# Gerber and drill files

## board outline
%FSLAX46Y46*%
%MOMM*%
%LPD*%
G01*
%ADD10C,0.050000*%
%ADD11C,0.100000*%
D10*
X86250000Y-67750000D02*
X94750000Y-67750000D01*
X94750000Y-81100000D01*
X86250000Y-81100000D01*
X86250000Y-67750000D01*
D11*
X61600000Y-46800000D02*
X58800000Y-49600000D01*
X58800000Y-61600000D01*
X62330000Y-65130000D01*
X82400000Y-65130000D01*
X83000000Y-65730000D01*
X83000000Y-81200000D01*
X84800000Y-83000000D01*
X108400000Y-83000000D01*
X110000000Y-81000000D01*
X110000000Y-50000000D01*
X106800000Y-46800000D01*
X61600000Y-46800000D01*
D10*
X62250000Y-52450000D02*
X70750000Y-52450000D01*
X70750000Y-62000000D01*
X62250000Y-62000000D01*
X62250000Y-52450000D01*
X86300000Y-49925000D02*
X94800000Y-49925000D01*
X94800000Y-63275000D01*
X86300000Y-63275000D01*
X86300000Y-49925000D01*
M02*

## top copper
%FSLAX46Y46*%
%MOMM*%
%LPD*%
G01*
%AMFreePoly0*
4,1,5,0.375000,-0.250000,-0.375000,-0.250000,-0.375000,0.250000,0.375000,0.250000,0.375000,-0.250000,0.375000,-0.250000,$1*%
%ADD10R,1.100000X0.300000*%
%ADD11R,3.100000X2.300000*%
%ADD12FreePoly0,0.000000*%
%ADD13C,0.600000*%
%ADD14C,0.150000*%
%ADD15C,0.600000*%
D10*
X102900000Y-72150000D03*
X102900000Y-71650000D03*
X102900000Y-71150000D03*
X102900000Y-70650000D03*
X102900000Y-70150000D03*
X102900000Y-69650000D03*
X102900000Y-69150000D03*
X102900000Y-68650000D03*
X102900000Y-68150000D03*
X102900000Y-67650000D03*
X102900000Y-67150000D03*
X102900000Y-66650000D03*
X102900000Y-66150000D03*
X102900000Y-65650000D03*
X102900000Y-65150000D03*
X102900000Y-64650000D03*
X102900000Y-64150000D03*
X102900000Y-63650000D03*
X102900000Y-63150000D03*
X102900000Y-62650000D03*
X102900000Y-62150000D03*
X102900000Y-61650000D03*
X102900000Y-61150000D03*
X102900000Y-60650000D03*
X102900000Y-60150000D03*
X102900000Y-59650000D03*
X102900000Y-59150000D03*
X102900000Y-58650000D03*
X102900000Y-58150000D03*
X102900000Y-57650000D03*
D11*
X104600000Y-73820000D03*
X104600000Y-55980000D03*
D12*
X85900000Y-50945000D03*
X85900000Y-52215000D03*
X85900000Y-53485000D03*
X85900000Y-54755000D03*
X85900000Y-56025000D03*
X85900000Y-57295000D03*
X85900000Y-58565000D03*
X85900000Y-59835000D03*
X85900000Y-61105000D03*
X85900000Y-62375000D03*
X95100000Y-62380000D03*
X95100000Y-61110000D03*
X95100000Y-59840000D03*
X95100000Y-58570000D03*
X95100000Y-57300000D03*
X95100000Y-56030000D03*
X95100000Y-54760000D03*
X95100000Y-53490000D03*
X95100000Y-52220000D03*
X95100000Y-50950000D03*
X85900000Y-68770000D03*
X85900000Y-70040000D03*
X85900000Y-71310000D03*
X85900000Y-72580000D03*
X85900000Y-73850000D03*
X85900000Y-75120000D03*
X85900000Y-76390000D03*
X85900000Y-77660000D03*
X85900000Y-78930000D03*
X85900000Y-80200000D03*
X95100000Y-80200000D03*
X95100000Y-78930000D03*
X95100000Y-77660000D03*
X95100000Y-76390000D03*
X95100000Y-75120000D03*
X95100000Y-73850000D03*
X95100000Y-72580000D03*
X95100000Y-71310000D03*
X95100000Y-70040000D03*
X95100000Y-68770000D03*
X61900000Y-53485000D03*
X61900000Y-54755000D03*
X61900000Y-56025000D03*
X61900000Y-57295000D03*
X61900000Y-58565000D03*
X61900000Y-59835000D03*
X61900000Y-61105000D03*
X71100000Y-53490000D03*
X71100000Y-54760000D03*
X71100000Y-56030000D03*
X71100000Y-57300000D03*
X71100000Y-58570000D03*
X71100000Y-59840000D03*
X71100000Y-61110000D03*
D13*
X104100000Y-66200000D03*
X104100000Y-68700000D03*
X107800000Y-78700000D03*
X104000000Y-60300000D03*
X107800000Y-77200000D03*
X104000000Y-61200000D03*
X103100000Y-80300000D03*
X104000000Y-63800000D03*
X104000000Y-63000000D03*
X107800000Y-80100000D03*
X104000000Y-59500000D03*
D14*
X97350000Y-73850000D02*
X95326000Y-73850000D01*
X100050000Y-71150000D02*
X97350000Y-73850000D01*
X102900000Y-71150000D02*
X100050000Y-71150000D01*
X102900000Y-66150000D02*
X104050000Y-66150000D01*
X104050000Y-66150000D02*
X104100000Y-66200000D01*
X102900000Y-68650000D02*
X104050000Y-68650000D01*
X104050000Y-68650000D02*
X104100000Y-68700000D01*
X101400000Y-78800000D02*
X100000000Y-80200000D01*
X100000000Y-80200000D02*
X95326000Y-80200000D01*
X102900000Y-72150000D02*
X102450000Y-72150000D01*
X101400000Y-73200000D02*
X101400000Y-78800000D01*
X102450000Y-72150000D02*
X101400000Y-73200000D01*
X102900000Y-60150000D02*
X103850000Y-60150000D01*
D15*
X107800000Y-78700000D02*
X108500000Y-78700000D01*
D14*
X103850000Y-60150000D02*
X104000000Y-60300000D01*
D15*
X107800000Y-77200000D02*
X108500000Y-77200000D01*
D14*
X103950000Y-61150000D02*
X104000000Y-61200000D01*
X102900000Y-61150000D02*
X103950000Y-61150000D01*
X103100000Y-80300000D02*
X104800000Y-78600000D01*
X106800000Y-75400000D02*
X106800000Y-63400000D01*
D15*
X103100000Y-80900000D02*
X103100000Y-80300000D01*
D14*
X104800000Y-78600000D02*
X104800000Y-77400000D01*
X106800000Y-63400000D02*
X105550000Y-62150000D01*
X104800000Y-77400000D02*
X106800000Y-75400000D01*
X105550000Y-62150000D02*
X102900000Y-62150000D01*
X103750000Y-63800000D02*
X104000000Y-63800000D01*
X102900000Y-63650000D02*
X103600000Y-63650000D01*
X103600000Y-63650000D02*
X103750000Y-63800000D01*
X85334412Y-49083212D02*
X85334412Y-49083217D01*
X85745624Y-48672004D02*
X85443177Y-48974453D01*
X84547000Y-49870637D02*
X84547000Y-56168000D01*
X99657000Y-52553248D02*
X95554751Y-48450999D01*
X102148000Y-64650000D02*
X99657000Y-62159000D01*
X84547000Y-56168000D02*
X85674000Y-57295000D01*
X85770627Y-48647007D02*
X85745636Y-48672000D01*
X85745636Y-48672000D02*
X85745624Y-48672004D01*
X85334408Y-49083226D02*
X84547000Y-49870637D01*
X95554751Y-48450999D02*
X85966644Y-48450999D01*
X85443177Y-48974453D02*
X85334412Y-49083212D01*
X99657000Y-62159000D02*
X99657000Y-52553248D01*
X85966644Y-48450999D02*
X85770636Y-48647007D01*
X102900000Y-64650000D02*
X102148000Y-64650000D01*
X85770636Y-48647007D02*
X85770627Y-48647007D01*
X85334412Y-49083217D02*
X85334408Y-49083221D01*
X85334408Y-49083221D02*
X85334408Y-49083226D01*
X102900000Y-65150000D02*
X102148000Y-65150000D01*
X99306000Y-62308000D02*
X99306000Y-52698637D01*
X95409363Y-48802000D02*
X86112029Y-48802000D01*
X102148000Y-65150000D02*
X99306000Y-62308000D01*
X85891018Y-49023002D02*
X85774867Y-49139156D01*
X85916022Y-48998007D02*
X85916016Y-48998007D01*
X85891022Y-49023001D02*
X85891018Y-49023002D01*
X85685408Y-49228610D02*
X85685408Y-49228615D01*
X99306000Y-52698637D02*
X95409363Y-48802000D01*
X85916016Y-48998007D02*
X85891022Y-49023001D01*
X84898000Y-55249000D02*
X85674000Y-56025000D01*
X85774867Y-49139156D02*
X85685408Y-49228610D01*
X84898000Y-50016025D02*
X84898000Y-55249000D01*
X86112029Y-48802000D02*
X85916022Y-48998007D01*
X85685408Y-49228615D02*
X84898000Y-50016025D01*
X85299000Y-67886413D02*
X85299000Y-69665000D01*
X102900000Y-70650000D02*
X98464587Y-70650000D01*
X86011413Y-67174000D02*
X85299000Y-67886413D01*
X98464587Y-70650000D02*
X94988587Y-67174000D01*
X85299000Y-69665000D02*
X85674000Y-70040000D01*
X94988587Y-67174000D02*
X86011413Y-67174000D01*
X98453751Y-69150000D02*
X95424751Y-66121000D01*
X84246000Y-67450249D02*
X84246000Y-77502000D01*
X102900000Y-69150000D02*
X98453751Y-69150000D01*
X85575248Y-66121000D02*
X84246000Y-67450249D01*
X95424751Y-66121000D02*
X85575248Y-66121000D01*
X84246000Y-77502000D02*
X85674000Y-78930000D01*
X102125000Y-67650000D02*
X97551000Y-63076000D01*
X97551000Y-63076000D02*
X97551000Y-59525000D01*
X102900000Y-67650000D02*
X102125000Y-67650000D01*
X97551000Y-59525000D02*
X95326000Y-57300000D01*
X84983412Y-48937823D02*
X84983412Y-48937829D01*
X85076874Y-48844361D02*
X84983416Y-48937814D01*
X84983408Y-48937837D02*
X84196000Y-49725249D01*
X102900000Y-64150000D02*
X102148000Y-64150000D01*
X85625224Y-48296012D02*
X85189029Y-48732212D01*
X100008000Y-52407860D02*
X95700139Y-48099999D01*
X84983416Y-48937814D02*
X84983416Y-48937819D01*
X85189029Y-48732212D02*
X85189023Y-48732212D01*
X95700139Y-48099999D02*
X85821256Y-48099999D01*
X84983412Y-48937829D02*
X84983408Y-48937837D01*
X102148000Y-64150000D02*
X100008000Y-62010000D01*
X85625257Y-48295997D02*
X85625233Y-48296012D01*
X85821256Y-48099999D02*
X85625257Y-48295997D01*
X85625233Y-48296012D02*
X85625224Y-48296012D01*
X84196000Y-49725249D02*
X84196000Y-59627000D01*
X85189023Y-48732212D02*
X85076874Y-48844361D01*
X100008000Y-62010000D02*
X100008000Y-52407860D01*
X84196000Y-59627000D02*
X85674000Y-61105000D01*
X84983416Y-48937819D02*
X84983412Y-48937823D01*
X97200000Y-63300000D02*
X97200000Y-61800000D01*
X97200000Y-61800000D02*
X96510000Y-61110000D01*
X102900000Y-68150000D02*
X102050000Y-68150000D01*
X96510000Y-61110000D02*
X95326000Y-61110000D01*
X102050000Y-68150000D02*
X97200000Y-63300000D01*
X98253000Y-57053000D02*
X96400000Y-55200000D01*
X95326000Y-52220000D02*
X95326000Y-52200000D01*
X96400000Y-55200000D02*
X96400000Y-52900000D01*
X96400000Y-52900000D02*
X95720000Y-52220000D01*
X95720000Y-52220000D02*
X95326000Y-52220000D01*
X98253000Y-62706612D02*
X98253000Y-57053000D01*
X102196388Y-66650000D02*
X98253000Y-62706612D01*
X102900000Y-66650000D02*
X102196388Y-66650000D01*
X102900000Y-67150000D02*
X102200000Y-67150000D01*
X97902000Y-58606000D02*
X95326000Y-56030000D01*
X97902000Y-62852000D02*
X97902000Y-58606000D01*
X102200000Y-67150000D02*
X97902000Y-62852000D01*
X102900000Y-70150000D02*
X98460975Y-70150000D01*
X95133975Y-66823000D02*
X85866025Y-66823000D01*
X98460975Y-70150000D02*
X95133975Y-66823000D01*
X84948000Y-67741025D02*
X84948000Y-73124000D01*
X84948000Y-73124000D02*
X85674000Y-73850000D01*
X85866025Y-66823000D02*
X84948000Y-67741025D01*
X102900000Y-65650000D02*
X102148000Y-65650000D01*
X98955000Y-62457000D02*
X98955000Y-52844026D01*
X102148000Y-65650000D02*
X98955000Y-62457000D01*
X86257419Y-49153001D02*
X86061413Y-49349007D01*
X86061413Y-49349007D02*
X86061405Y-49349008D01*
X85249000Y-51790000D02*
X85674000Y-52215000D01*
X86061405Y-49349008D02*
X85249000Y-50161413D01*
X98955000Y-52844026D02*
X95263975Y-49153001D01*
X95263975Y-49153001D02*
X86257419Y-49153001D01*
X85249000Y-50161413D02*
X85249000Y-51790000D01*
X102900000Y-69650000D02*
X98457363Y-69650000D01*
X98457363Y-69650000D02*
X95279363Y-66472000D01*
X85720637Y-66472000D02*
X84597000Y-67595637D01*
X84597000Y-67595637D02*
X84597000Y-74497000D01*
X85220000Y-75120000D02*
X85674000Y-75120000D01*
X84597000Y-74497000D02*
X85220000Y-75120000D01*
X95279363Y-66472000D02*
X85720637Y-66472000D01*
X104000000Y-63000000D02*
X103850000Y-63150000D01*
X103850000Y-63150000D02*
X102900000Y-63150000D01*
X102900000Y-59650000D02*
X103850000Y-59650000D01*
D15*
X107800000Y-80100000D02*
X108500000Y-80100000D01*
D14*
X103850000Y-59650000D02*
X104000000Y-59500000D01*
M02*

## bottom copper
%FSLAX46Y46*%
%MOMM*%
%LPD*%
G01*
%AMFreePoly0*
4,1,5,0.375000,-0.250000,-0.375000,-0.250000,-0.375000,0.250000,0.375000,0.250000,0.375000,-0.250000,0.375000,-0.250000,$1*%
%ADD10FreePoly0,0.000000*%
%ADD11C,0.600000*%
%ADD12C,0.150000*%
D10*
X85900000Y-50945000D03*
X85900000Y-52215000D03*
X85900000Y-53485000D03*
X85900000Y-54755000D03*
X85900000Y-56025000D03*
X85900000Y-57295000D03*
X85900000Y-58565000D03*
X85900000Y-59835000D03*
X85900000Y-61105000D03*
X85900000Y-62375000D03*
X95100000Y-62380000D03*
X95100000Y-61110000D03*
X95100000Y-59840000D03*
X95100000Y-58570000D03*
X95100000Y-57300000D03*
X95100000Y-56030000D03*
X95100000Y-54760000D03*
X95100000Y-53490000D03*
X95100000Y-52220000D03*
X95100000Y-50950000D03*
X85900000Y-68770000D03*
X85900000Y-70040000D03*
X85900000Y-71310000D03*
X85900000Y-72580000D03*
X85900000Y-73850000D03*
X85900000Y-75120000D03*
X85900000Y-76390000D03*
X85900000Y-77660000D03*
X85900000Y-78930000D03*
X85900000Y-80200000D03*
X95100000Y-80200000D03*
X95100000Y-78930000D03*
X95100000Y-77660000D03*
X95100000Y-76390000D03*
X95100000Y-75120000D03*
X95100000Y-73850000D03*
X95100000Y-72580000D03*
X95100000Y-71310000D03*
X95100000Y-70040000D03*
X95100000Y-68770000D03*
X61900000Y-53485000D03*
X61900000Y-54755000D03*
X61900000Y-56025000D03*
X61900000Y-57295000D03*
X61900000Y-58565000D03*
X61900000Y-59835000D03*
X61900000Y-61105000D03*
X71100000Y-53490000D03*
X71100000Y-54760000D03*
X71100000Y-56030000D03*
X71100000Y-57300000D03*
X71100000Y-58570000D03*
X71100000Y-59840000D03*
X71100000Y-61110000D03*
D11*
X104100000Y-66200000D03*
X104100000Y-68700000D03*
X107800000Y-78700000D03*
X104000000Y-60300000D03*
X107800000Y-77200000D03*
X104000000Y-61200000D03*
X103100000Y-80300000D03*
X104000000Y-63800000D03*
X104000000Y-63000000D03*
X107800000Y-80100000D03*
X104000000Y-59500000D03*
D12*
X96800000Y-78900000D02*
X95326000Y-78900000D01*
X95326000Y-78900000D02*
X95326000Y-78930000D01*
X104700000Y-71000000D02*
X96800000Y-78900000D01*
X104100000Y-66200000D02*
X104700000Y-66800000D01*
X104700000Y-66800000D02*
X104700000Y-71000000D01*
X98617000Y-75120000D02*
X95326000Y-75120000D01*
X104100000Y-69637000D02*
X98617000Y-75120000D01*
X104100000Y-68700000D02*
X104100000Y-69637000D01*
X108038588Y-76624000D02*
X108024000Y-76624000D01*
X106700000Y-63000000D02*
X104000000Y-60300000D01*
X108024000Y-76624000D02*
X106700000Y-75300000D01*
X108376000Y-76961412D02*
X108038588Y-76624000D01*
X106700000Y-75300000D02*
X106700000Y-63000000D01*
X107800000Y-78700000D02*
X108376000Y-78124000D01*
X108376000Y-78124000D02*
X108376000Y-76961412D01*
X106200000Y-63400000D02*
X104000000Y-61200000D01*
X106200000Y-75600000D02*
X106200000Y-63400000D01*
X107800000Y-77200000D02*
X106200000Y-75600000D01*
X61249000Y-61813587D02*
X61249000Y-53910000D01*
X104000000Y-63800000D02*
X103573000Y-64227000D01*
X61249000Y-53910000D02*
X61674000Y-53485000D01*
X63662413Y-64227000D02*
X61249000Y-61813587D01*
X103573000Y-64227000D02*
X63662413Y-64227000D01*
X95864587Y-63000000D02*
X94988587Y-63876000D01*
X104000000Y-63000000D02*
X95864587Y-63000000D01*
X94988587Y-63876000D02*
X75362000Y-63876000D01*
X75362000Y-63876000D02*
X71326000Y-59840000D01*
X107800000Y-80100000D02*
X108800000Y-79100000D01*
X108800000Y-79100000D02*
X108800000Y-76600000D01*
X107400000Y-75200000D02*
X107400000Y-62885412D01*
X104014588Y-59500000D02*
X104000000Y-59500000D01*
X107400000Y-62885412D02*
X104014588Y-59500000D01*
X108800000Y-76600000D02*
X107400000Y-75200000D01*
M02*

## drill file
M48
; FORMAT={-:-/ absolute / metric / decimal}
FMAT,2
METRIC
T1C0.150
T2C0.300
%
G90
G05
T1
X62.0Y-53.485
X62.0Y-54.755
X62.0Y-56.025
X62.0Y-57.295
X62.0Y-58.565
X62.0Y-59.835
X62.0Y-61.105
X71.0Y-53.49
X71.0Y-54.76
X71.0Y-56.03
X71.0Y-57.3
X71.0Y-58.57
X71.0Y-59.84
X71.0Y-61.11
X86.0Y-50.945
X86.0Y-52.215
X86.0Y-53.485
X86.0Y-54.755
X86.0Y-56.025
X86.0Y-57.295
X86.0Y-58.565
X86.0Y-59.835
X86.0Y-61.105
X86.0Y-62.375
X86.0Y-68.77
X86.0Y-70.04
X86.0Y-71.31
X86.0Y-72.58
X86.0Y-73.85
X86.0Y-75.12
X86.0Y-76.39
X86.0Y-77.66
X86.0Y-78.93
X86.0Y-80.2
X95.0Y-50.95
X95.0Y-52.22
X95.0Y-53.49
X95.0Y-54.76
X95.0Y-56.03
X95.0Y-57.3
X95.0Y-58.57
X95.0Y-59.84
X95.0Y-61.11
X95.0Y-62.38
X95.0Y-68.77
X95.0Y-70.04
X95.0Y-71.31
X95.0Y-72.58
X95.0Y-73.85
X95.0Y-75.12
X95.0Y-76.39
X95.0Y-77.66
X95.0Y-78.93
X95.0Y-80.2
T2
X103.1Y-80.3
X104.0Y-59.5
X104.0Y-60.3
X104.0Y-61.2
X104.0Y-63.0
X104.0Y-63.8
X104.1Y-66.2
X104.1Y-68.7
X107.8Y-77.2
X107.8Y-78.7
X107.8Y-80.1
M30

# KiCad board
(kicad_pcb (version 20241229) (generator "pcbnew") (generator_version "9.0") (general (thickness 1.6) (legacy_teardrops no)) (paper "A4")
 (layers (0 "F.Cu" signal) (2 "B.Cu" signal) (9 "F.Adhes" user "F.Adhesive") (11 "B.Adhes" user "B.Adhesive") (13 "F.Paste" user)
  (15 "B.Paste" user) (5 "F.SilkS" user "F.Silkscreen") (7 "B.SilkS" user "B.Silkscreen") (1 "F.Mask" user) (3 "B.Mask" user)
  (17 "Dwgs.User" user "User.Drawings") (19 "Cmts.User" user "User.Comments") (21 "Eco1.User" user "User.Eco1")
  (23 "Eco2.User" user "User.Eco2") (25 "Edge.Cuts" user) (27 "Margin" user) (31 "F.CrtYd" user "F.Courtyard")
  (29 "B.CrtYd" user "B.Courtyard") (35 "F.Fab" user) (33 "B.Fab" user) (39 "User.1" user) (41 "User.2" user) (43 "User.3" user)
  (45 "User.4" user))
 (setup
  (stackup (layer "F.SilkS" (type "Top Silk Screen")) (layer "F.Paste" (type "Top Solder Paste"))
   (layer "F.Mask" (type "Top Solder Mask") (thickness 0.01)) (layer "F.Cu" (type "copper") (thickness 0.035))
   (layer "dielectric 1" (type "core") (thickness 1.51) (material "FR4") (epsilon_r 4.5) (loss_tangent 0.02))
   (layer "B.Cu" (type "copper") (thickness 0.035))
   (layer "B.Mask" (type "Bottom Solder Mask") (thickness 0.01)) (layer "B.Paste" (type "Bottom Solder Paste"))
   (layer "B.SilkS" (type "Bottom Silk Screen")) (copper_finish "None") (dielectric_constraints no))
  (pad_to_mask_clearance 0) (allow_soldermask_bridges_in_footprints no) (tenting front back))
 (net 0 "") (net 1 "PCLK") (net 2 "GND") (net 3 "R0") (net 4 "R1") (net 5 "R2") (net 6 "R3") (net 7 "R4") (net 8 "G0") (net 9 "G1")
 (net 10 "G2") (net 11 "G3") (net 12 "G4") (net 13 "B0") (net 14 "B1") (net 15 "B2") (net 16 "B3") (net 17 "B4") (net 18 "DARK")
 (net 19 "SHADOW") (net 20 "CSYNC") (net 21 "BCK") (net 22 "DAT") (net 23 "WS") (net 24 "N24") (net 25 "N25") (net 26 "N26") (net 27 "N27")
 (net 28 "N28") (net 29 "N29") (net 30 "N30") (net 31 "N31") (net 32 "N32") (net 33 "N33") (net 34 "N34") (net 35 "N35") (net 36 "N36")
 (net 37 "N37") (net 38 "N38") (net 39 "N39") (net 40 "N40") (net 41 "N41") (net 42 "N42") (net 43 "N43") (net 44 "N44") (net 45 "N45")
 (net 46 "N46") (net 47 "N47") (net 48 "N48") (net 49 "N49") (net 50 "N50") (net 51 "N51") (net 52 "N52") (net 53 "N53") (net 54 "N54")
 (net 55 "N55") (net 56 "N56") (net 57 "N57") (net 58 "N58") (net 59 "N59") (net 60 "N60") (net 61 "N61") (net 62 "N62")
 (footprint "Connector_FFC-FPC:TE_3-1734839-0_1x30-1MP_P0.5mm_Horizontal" (layer "F.Cu") (at 104.25 64.9 90)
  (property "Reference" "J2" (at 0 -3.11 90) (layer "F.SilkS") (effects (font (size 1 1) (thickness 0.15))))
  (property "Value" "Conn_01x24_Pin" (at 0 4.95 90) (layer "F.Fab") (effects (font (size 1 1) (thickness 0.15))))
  (pad "1" smd rect (at -7.25 -1.35 90) (size 0.3 1.1) (layers "F.Cu" "F.Mask" "F.Paste") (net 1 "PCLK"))
  (pad "2" smd rect (at -6.75 -1.35 90) (size 0.3 1.1) (layers "F.Cu" "F.Mask" "F.Paste") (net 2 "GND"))
  (pad "3" smd rect (at -6.25 -1.35 90) (size 0.3 1.1) (layers "F.Cu" "F.Mask" "F.Paste") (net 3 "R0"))
  (pad "4" smd rect (at -5.75 -1.35 90) (size 0.3 1.1) (layers "F.Cu" "F.Mask" "F.Paste") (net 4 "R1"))
  (pad "5" smd rect (at -5.25 -1.35 90) (size 0.3 1.1) (layers "F.Cu" "F.Mask" "F.Paste") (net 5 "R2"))
  (pad "6" smd rect (at -4.75 -1.35 90) (size 0.3 1.1) (layers "F.Cu" "F.Mask" "F.Paste") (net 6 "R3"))
  (pad "7" smd rect (at -4.25 -1.35 90) (size 0.3 1.1) (layers "F.Cu" "F.Mask" "F.Paste") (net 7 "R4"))
  (pad "8" smd rect (at -3.75 -1.35 90) (size 0.3 1.1) (layers "F.Cu" "F.Mask" "F.Paste") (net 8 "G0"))
  (pad "9" smd rect (at -3.25 -1.35 90) (size 0.3 1.1) (layers "F.Cu" "F.Mask" "F.Paste") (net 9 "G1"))
  (pad "10" smd rect (at -2.75 -1.35 90) (size 0.3 1.1) (layers "F.Cu" "F.Mask" "F.Paste") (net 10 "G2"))
  (pad "11" smd rect (at -2.25 -1.35 90) (size 0.3 1.1) (layers "F.Cu" "F.Mask" "F.Paste") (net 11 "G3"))
  (pad "12" smd rect (at -1.75 -1.35 90) (size 0.3 1.1) (layers "F.Cu" "F.Mask" "F.Paste") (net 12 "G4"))
  (pad "13" smd rect (at -1.25 -1.35 90) (size 0.3 1.1) (layers "F.Cu" "F.Mask" "F.Paste") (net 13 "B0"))
  (pad "14" smd rect (at -0.75 -1.35 90) (size 0.3 1.1) (layers "F.Cu" "F.Mask" "F.Paste") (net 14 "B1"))
  (pad "15" smd rect (at -0.25 -1.35 90) (size 0.3 1.1) (layers "F.Cu" "F.Mask" "F.Paste") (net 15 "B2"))
  (pad "16" smd rect (at 0.25 -1.35 90) (size 0.3 1.1) (layers "F.Cu" "F.Mask" "F.Paste") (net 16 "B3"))
  (pad "17" smd rect (at 0.75 -1.35 90) (size 0.3 1.1) (layers "F.Cu" "F.Mask" "F.Paste") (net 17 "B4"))
  (pad "18" smd rect (at 1.25 -1.35 90) (size 0.3 1.1) (layers "F.Cu" "F.Mask" "F.Paste") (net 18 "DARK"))
  (pad "19" smd rect (at 1.75 -1.35 90) (size 0.3 1.1) (layers "F.Cu" "F.Mask" "F.Paste") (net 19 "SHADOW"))
  (pad "20" smd rect (at 2.25 -1.35 90) (size 0.3 1.1) (layers "F.Cu" "F.Mask" "F.Paste") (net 2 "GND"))
  (pad "21" smd rect (at 2.75 -1.35 90) (size 0.3 1.1) (layers "F.Cu" "F.Mask" "F.Paste") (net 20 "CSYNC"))
  (pad "22" smd rect (at 3.25 -1.35 90) (size 0.3 1.1) (layers "F.Cu" "F.Mask" "F.Paste") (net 2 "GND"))
  (pad "23" smd rect (at 3.75 -1.35 90) (size 0.3 1.1) (layers "F.Cu" "F.Mask" "F.Paste") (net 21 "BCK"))
  (pad "24" smd rect (at 4.25 -1.35 90) (size 0.3 1.1) (layers "F.Cu" "F.Mask" "F.Paste") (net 2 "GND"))
  (pad "25" smd rect (at 4.75 -1.35 90) (size 0.3 1.1) (layers "F.Cu" "F.Mask" "F.Paste") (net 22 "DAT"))
  (pad "26" smd rect (at 5.25 -1.35 90) (size 0.3 1.1) (layers "F.Cu" "F.Mask" "F.Paste") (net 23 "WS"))
  (pad "27" smd rect (at 5.75 -1.35 90) (size 0.3 1.1) (layers "F.Cu" "F.Mask" "F.Paste") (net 2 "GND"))
  (pad "28" smd rect (at 6.25 -1.35 90) (size 0.3 1.1) (layers "F.Cu" "F.Mask" "F.Paste") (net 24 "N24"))
  (pad "29" smd rect (at 6.75 -1.35 90) (size 0.3 1.1) (layers "F.Cu" "F.Mask" "F.Paste") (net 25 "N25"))
  (pad "30" smd rect (at 7.25 -1.35 90) (size 0.3 1.1) (layers "F.Cu" "F.Mask" "F.Paste") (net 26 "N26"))
  (pad "MP" smd rect (at -8.92 0.35 90) (size 2.3 3.1) (layers "F.Cu" "F.Mask" "F.Paste"))
  (pad "MP" smd rect (at 8.92 0.35 90) (size 2.3 3.1) (layers "F.Cu" "F.Mask" "F.Paste")))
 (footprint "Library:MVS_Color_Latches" (layer "F.Cu") (at 77.8 65.43)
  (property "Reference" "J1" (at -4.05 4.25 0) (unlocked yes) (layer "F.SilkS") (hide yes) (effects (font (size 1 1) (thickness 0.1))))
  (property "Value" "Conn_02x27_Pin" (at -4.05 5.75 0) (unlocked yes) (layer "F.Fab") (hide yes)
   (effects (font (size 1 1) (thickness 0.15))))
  (pad "1" thru_hole custom (at 8.2 -14.485) (size 0.75 0.5) (drill 0.15 (offset -0.1 0)) (layers "*.Cu" "*.Mask") (remove_unused_layers no)
   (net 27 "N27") (options (clearance outline) (anchor rect)) (primitives))
  (pad "2" thru_hole custom (at 8.2 -13.215) (size 0.75 0.5) (drill 0.15 (offset -0.1 0)) (layers "*.Cu" "*.Mask") (remove_unused_layers no)
   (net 14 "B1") (options (clearance outline) (anchor rect)) (primitives))
  (pad "3" thru_hole custom (at 8.2 -11.945) (size 0.75 0.5) (drill 0.15 (offset -0.1 0)) (layers "*.Cu" "*.Mask") (remove_unused_layers no)
   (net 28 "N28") (options (clearance outline) (anchor rect)) (primitives))
  (pad "4" thru_hole custom (at 8.2 -10.675) (size 0.75 0.5) (drill 0.15 (offset -0.1 0)) (layers "*.Cu" "*.Mask") (remove_unused_layers no)
   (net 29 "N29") (options (clearance outline) (anchor rect)) (primitives))
  (pad "5" thru_hole custom (at 8.2 -9.405) (size 0.75 0.5) (drill 0.15 (offset -0.1 0)) (layers "*.Cu" "*.Mask") (remove_unused_layers no)
   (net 15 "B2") (options (clearance outline) (anchor rect)) (primitives))
  (pad "6" thru_hole custom (at 8.2 -8.135) (size 0.75 0.5) (drill 0.15 (offset -0.1 0)) (layers "*.Cu" "*.Mask") (remove_unused_layers no)
   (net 16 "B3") (options (clearance outline) (anchor rect)) (primitives))
  (pad "7" thru_hole custom (at 8.2 -6.865) (size 0.75 0.5) (drill 0.15 (offset -0.1 0)) (layers "*.Cu" "*.Mask") (remove_unused_layers no)
   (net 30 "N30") (options (clearance outline) (anchor rect)) (primitives))
  (pad "8" thru_hole custom (at 8.2 -5.595) (size 0.75 0.5) (drill 0.15 (offset -0.1 0)) (layers "*.Cu" "*.Mask") (remove_unused_layers no)
   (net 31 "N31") (options (clearance outline) (anchor rect)) (primitives))
  (pad "9" thru_hole custom (at 8.2 -4.325) (size 0.75 0.5) (drill 0.15 (offset -0.1 0)) (layers "*.Cu" "*.Mask") (remove_unused_layers no)
   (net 17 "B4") (options (clearance outline) (anchor rect)) (primitives))
  (pad "10" thru_hole custom (at 8.2 -3.055) (size 0.75 0.5) (drill 0.15 (offset -0.1 0)) (layers "*.Cu" "*.Mask") (remove_unused_layers no)
   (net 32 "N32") (options (clearance outline) (anchor rect)) (primitives))
  (pad "11" thru_hole custom (at 17.2 -3.05) (size 0.75 0.5) (drill 0.15 (offset 0.1 0)) (layers "*.Cu" "*.Mask") (remove_unused_layers no)
   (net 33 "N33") (options (clearance outline) (anchor rect)) (primitives))
  (pad "12" thru_hole custom (at 17.2 -4.32) (size 0.75 0.5) (drill 0.15 (offset 0.1 0)) (layers "*.Cu" "*.Mask") (remove_unused_layers no)
   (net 9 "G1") (options (clearance outline) (anchor rect)) (primitives))
  (pad "13" thru_hole custom (at 17.2 -5.59) (size 0.75 0.5) (drill 0.15 (offset 0.1 0)) (layers "*.Cu" "*.Mask") (remove_unused_layers no)
   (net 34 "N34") (options (clearance outline) (anchor rect)) (primitives))
  (pad "14" thru_hole custom (at 17.2 -6.86) (size 0.75 0.5) (drill 0.15 (offset 0.1 0)) (layers "*.Cu" "*.Mask") (remove_unused_layers no)
   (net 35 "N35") (options (clearance outline) (anchor rect)) (primitives))
  (pad "15" thru_hole custom (at 17.2 -8.13) (size 0.75 0.5) (drill 0.15 (offset 0.1 0)) (layers "*.Cu" "*.Mask") (remove_unused_layers no)
   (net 10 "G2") (options (clearance outline) (anchor rect)) (primitives))
  (pad "16" thru_hole custom (at 17.2 -9.4) (size 0.75 0.5) (drill 0.15 (offset 0.1 0)) (layers "*.Cu" "*.Mask") (remove_unused_layers no)
   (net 11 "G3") (options (clearance outline) (anchor rect)) (primitives))
  (pad "17" thru_hole custom (at 17.2 -10.67) (size 0.75 0.5) (drill 0.15 (offset 0.1 0)) (layers "*.Cu" "*.Mask") (remove_unused_layers no)
   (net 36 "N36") (options (clearance outline) (anchor rect)) (primitives))
  (pad "18" thru_hole custom (at 17.2 -11.94) (size 0.75 0.5) (drill 0.15 (offset 0.1 0)) (layers "*.Cu" "*.Mask") (remove_unused_layers no)
   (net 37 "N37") (options (clearance outline) (anchor rect)) (primitives))
  (pad "19" thru_hole custom (at 17.2 -13.21) (size 0.75 0.5) (drill 0.15 (offset 0.1 0)) (layers "*.Cu" "*.Mask") (remove_unused_layers no)
   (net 12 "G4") (options (clearance outline) (anchor rect)) (primitives))
  (pad "20" thru_hole custom (at 17.2 -14.48) (size 0.75 0.5) (drill 0.15 (offset 0.1 0)) (layers "*.Cu" "*.Mask") (remove_unused_layers no)
   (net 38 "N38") (options (clearance outline) (anchor rect)) (primitives))
  (pad "21" thru_hole custom (at 8.2 3.34) (size 0.75 0.5) (drill 0.15 (offset -0.1 0)) (layers "*.Cu" "*.Mask") (remove_unused_layers no)
   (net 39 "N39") (options (clearance outline) (anchor rect)) (primitives))
  (pad "22" thru_hole custom (at 8.2 4.61) (size 0.75 0.5) (drill 0.15 (offset -0.1 0)) (layers "*.Cu" "*.Mask") (remove_unused_layers no)
   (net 4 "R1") (options (clearance outline) (anchor rect)) (primitives))
  (pad "23" thru_hole custom (at 8.2 5.88) (size 0.75 0.5) (drill 0.15 (offset -0.1 0)) (layers "*.Cu" "*.Mask") (remove_unused_layers no)
   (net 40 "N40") (options (clearance outline) (anchor rect)) (primitives))
  (pad "24" thru_hole custom (at 8.2 7.15) (size 0.75 0.5) (drill 0.15 (offset -0.1 0)) (layers "*.Cu" "*.Mask") (remove_unused_layers no)
   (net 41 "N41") (options (clearance outline) (anchor rect)) (primitives))
  (pad "25" thru_hole custom (at 8.2 8.42) (size 0.75 0.5) (drill 0.15 (offset -0.1 0)) (layers "*.Cu" "*.Mask") (remove_unused_layers no)
   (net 5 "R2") (options (clearance outline) (anchor rect)) (primitives))
  (pad "26" thru_hole custom (at 8.2 9.69) (size 0.75 0.5) (drill 0.15 (offset -0.1 0)) (layers "*.Cu" "*.Mask") (remove_unused_layers no)
   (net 6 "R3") (options (clearance outline) (anchor rect)) (primitives))
  (pad "27" thru_hole custom (at 8.2 10.96) (size 0.75 0.5) (drill 0.15 (offset -0.1 0)) (layers "*.Cu" "*.Mask") (remove_unused_layers no)
   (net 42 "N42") (options (clearance outline) (anchor rect)) (primitives))
  (pad "28" thru_hole custom (at 8.2 12.23) (size 0.75 0.5) (drill 0.15 (offset -0.1 0)) (layers "*.Cu" "*.Mask") (remove_unused_layers no)
   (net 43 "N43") (options (clearance outline) (anchor rect)) (primitives))
  (pad "29" thru_hole custom (at 8.2 13.5) (size 0.75 0.5) (drill 0.15 (offset -0.1 0)) (layers "*.Cu" "*.Mask") (remove_unused_layers no)
   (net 7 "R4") (options (clearance outline) (anchor rect)) (primitives))
  (pad "30" thru_hole custom (at 8.2 14.77) (size 0.75 0.5) (drill 0.15 (offset -0.1 0)) (layers "*.Cu" "*.Mask") (remove_unused_layers no)
   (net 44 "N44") (options (clearance outline) (anchor rect)) (primitives))
  (pad "31" thru_hole custom (at 17.2 14.77) (size 0.75 0.5) (drill 0.15 (offset 0.1 0)) (layers "*.Cu" "*.Mask") (remove_unused_layers no)
   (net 1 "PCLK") (options (clearance outline) (anchor rect)) (primitives))
  (pad "32" thru_hole custom (at 17.2 13.5) (size 0.75 0.5) (drill 0.15 (offset 0.1 0)) (layers "*.Cu" "*.Mask") (remove_unused_layers no)
   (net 13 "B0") (options (clearance outline) (anchor rect)) (primitives))
  (pad "33" thru_hole custom (at 17.2 12.23) (size 0.75 0.5) (drill 0.15 (offset 0.1 0)) (layers "*.Cu" "*.Mask") (remove_unused_layers no)
   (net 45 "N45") (options (clearance outline) (anchor rect)) (primitives))
  (pad "34" thru_hole custom (at 17.2 10.96) (size 0.75 0.5) (drill 0.15 (offset 0.1 0)) (layers "*.Cu" "*.Mask") (remove_unused_layers no)
   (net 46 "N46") (options (clearance outline) (anchor rect)) (primitives))
  (pad "35" thru_hole custom (at 17.2 9.69) (size 0.75 0.5) (drill 0.15 (offset 0.1 0)) (layers "*.Cu" "*.Mask") (remove_unused_layers no)
   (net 8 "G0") (options (clearance outline) (anchor rect)) (primitives))
  (pad "36" thru_hole custom (at 17.2 8.42) (size 0.75 0.5) (drill 0.15 (offset 0.1 0)) (layers "*.Cu" "*.Mask") (remove_unused_layers no)
   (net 3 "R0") (options (clearance outline) (anchor rect)) (primitives))
  (pad "37" thru_hole custom (at 17.2 7.15) (size 0.75 0.5) (drill 0.15 (offset 0.1 0)) (layers "*.Cu" "*.Mask") (remove_unused_layers no)
   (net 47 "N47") (options (clearance outline) (anchor rect)) (primitives))
  (pad "38" thru_hole custom (at 17.2 5.88) (size 0.75 0.5) (drill 0.15 (offset 0.1 0)) (layers "*.Cu" "*.Mask") (remove_unused_layers no)
   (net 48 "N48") (options (clearance outline) (anchor rect)) (primitives))
  (pad "39" thru_hole custom (at 17.2 4.61) (size 0.75 0.5) (drill 0.15 (offset 0.1 0)) (layers "*.Cu" "*.Mask") (remove_unused_layers no)
   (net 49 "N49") (options (clearance outline) (anchor rect)) (primitives))
  (pad "40" thru_hole custom (at 17.2 3.34) (size 0.75 0.5) (drill 0.15 (offset 0.1 0)) (layers "*.Cu" "*.Mask") (remove_unused_layers no)
   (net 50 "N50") (options (clearance outline) (anchor rect)) (primitives))
  (pad "41" thru_hole custom (at -15.8 -11.945) (size 0.75 0.5) (drill 0.15 (offset -0.1 0)) (layers "*.Cu" "*.Mask")
   (remove_unused_layers no) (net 18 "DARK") (options (clearance outline) (anchor rect)) (primitives))
  (pad "42" thru_hole custom (at -15.8 -10.675) (size 0.75 0.5) (drill 0.15 (offset -0.1 0)) (layers "*.Cu" "*.Mask")
   (remove_unused_layers no) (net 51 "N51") (options (clearance outline) (anchor rect)) (primitives))
  (pad "43" thru_hole custom (at -15.8 -9.405) (size 0.75 0.5) (drill 0.15 (offset -0.1 0)) (layers "*.Cu" "*.Mask")
   (remove_unused_layers no) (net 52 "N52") (options (clearance outline) (anchor rect)) (primitives))
  (pad "44" thru_hole custom (at -15.8 -8.135) (size 0.75 0.5) (drill 0.15 (offset -0.1 0)) (layers "*.Cu" "*.Mask")
   (remove_unused_layers no) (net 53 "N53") (options (clearance outline) (anchor rect)) (primitives))
  (pad "45" thru_hole custom (at -15.8 -6.865) (size 0.75 0.5) (drill 0.15 (offset -0.1 0)) (layers "*.Cu" "*.Mask")
   (remove_unused_layers no) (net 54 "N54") (options (clearance outline) (anchor rect)) (primitives))
  (pad "46" thru_hole custom (at -15.8 -5.595) (size 0.75 0.5) (drill 0.15 (offset -0.1 0)) (layers "*.Cu" "*.Mask")
   (remove_unused_layers no) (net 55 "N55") (options (clearance outline) (anchor rect)) (primitives))
  (pad "47" thru_hole custom (at -15.8 -4.325) (size 0.75 0.5) (drill 0.15 (offset -0.1 0)) (layers "*.Cu" "*.Mask")
   (remove_unused_layers no) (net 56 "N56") (options (clearance outline) (anchor rect)) (primitives))
  (pad "48" thru_hole custom (at -6.8 -11.94) (size 0.75 0.5) (drill 0.15 (offset 0.1 0)) (layers "*.Cu" "*.Mask") (remove_unused_layers no)
   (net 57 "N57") (options (clearance outline) (anchor rect)) (primitives))
  (pad "49" thru_hole custom (at -6.8 -10.67) (size 0.75 0.5) (drill 0.15 (offset 0.1 0)) (layers "*.Cu" "*.Mask") (remove_unused_layers no)
   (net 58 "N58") (options (clearance outline) (anchor rect)) (primitives))
  (pad "50" thru_hole custom (at -6.8 -9.4) (size 0.75 0.5) (drill 0.15 (offset 0.1 0)) (layers "*.Cu" "*.Mask") (remove_unused_layers no)
   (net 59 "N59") (options (clearance outline) (anchor rect)) (primitives))
  (pad "51" thru_hole custom (at -6.8 -8.13) (size 0.75 0.5) (drill 0.15 (offset 0.1 0)) (layers "*.Cu" "*.Mask") (remove_unused_layers no)
   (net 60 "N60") (options (clearance outline) (anchor rect)) (primitives))
  (pad "52" thru_hole custom (at -6.8 -6.86) (size 0.75 0.5) (drill 0.15 (offset 0.1 0)) (layers "*.Cu" "*.Mask") (remove_unused_layers no)
   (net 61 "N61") (options (clearance outline) (anchor rect)) (primitives))
  (pad "53" thru_hole custom (at -6.8 -5.59) (size 0.75 0.5) (drill 0.15 (offset 0.1 0)) (layers "*.Cu" "*.Mask") (remove_unused_layers no)
   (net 19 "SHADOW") (options (clearance outline) (anchor rect)) (primitives))
  (pad "54" thru_hole custom (at -6.8 -4.32) (size 0.75 0.5) (drill 0.15 (offset 0.1 0)) (layers "*.Cu" "*.Mask") (remove_unused_layers no)
   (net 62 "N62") (options (clearance outline) (anchor rect)) (primitives)))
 (gr_rect (start 86.25 67.75) (end 94.75 81.1) (stroke (width 0.05) (type default)) (fill no) (layer "Edge.Cuts"))
 (gr_poly
  (pts (xy 61.6 46.8) (xy 58.8 49.6) (xy 58.8 61.6) (xy 62.33 65.13) (xy 82.4 65.13) (xy 83 65.73) (xy 83 81.2) (xy 84.8 83) (xy 108.4 83)
   (xy 110 81) (xy 110 50) (xy 106.8 46.8))
  (stroke (width 0.1) (type solid)) (fill no) (layer "Edge.Cuts"))
 (gr_rect (start 62.25 52.45) (end 70.75 62) (stroke (width 0.05) (type default)) (fill no) (layer "Edge.Cuts"))
 (gr_rect (start 86.3 49.925) (end 94.8 63.275) (stroke (width 0.05) (type default)) (fill no) (layer "Edge.Cuts"))
 (segment (start 97.35 73.85) (end 95.326 73.85) (width 0.15) (layer "F.Cu") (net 3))
 (segment (start 100.05 71.15) (end 97.35 73.85) (width 0.15) (layer "F.Cu") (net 3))
 (segment (start 102.9 71.15) (end 100.05 71.15) (width 0.15) (layer "F.Cu") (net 3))
 (segment (start 102.9 66.15) (end 104.05 66.15) (width 0.15) (layer "F.Cu") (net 13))
 (segment (start 104.05 66.15) (end 104.1 66.2) (width 0.15) (layer "F.Cu") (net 13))
 (via (at 104.1 66.2) (size 0.6) (drill 0.3) (layers "F.Cu" "B.Cu") (free yes) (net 13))
 (segment (start 96.8 78.9) (end 95.326 78.9) (width 0.15) (layer "B.Cu") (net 13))
 (segment (start 95.326 78.9) (end 95.326 78.93) (width 0.15) (layer "B.Cu") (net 13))
 (segment (start 104.7 71) (end 96.8 78.9) (width 0.15) (layer "B.Cu") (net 13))
 (segment (start 104.1 66.2) (end 104.7 66.8) (width 0.15) (layer "B.Cu") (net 13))
 (segment (start 104.7 66.8) (end 104.7 71) (width 0.15) (layer "B.Cu") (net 13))
 (segment (start 102.9 68.65) (end 104.05 68.65) (width 0.15) (layer "F.Cu") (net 8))
 (segment (start 104.05 68.65) (end 104.1 68.7) (width 0.15) (layer "F.Cu") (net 8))
 (via (at 104.1 68.7) (size 0.6) (drill 0.3) (layers "F.Cu" "B.Cu") (free yes) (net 8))
 (segment (start 98.617 75.12) (end 95.326 75.12) (width 0.15) (layer "B.Cu") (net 8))
 (segment (start 104.1 69.637) (end 98.617 75.12) (width 0.15) (layer "B.Cu") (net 8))
 (segment (start 104.1 68.7) (end 104.1 69.637) (width 0.15) (layer "B.Cu") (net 8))
 (segment (start 101.4 78.8) (end 100 80.2) (width 0.15) (layer "F.Cu") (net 1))
 (segment (start 100 80.2) (end 95.326 80.2) (width 0.15) (layer "F.Cu") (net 1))
 (segment (start 102.9 72.15) (end 102.45 72.15) (width 0.15) (layer "F.Cu") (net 1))
 (segment (start 101.4 73.2) (end 101.4 78.8) (width 0.15) (layer "F.Cu") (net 1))
 (segment (start 102.45 72.15) (end 101.4 73.2) (width 0.15) (layer "F.Cu") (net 1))
 (segment (start 102.9 60.15) (end 103.85 60.15) (width 0.15) (layer "F.Cu") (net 22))
 (segment (start 107.8 78.7) (end 108.5 78.7) (width 0.6) (layers "F.Cu" "F.Mask") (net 22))
 (segment (start 103.85 60.15) (end 104 60.3) (width 0.15) (layer "F.Cu") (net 22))
 (via (at 107.8 78.7) (size 0.6) (drill 0.3) (layers "F.Cu" "B.Cu") (free yes) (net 22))
 (via (at 104 60.3) (size 0.6) (drill 0.3) (layers "F.Cu" "B.Cu") (free yes) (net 22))
 (segment (start 108.038588 76.624) (end 108.024 76.624) (width 0.15) (layer "B.Cu") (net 22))
 (segment (start 106.7 63) (end 104 60.3) (width 0.15) (layer "B.Cu") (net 22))
 (segment (start 108.024 76.624) (end 106.7 75.3) (width 0.15) (layer "B.Cu") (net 22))
 (segment (start 108.376 76.961412) (end 108.038588 76.624) (width 0.15) (layer "B.Cu") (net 22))
 (segment (start 106.7 75.3) (end 106.7 63) (width 0.15) (layer "B.Cu") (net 22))
 (segment (start 107.8 78.7) (end 108.376 78.124) (width 0.15) (layer "B.Cu") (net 22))
 (segment (start 108.376 78.124) (end 108.376 76.961412) (width 0.15) (layer "B.Cu") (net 22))
 (segment (start 107.8 77.2) (end 108.5 77.2) (width 0.6) (layers "F.Cu" "F.Mask") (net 21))
 (segment (start 103.95 61.15) (end 104 61.2) (width 0.15) (layer "F.Cu") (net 21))
 (segment (start 102.9 61.15) (end 103.95 61.15) (width 0.15) (layer "F.Cu") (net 21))
 (via (at 107.8 77.2) (size 0.6) (drill 0.3) (layers "F.Cu" "B.Cu") (free yes) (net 21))
 (via (at 104 61.2) (size 0.6) (drill 0.3) (layers "F.Cu" "B.Cu") (free yes) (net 21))
 (segment (start 106.2 63.4) (end 104 61.2) (width 0.15) (layer "B.Cu") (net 21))
 (segment (start 106.2 75.6) (end 106.2 63.4) (width 0.15) (layer "B.Cu") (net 21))
 (segment (start 107.8 77.2) (end 106.2 75.6) (width 0.15) (layer "B.Cu") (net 21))
 (segment (start 103.1 80.3) (end 104.8 78.6) (width 0.15) (layer "F.Cu") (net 20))
 (segment (start 106.8 75.4) (end 106.8 63.4) (width 0.15) (layer "F.Cu") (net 20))
 (segment (start 103.1 80.9) (end 103.1 80.3) (width 0.6) (layer "F.Cu") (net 20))
 (segment (start 104.8 78.6) (end 104.8 77.4) (width 0.15) (layer "F.Cu") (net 20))
 (segment (start 106.8 63.4) (end 105.55 62.15) (width 0.15) (layer "F.Cu") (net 20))
 (segment (start 104.8 77.4) (end 106.8 75.4) (width 0.15) (layer "F.Cu") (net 20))
 (segment (start 105.55 62.15) (end 102.9 62.15) (width 0.15) (layer "F.Cu") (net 20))
 (via (at 103.1 80.3) (size 0.6) (drill 0.3) (layers "F.Cu" "B.Cu") (free yes) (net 20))
 (segment (start 103.75 63.8) (end 104 63.8) (width 0.15) (layer "F.Cu") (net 18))
 (segment (start 102.9 63.65) (end 103.6 63.65) (width 0.15) (layer "F.Cu") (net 18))
 (segment (start 103.6 63.65) (end 103.75 63.8) (width 0.15) (layer "F.Cu") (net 18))
 (via (at 104 63.8) (size 0.6) (drill 0.3) (layers "F.Cu" "B.Cu") (free yes) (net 18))
 (segment (start 61.249 61.813587) (end 61.249 53.91) (width 0.15) (layer "B.Cu") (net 18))
 (segment (start 104 63.8) (end 103.573 64.227) (width 0.15) (layer "B.Cu") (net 18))
 (segment (start 61.249 53.91) (end 61.674 53.485) (width 0.15) (layer "B.Cu") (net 18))
 (segment (start 63.662413 64.227) (end 61.249 61.813587) (width 0.15) (layer "B.Cu") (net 18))
 (segment (start 103.573 64.227) (end 63.662413 64.227) (width 0.15) (layer "B.Cu") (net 18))
 (segment (start 85.334412 49.083212) (end 85.334412 49.083217) (width 0.15) (layer "F.Cu") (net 16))
 (segment (start 85.745624 48.672004) (end 85.443177 48.974453) (width 0.15) (layer "F.Cu") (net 16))
 (segment (start 84.547 49.870637) (end 84.547 56.168) (width 0.15) (layer "F.Cu") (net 16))
 (segment (start 99.657 52.553248) (end 95.554751 48.450999) (width 0.15) (layer "F.Cu") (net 16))
 (segment (start 102.148 64.65) (end 99.657 62.159) (width 0.15) (layer "F.Cu") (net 16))
 (segment (start 84.547 56.168) (end 85.674 57.295) (width 0.15) (layer "F.Cu") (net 16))
 (segment (start 85.770627 48.647007) (end 85.745636 48.672) (width 0.15) (layer "F.Cu") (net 16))
 (segment (start 85.745636 48.672) (end 85.745624 48.672004) (width 0.15) (layer "F.Cu") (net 16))
 (segment (start 85.334408 49.083226) (end 84.547 49.870637) (width 0.15) (layer "F.Cu") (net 16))
 (segment (start 95.554751 48.450999) (end 85.966644 48.450999) (width 0.15) (layer "F.Cu") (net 16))
 (segment (start 85.443177 48.974453) (end 85.334412 49.083212) (width 0.15) (layer "F.Cu") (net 16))
 (segment (start 99.657 62.159) (end 99.657 52.553248) (width 0.15) (layer "F.Cu") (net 16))
 (segment (start 85.966644 48.450999) (end 85.770636 48.647007) (width 0.15) (layer "F.Cu") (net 16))
 (segment (start 102.9 64.65) (end 102.148 64.65) (width 0.15) (layer "F.Cu") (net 16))
 (segment (start 85.770636 48.647007) (end 85.770627 48.647007) (width 0.15) (layer "F.Cu") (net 16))
 (segment (start 85.334412 49.083217) (end 85.334408 49.083221) (width 0.15) (layer "F.Cu") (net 16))
 (segment (start 85.334408 49.083221) (end 85.334408 49.083226) (width 0.15) (layer "F.Cu") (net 16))
 (segment (start 102.9 65.15) (end 102.148 65.15) (width 0.15) (layer "F.Cu") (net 15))
 (segment (start 99.306 62.308) (end 99.306 52.698637) (width 0.15) (layer "F.Cu") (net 15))
 (segment (start 95.409363 48.802) (end 86.112029 48.802) (width 0.15) (layer "F.Cu") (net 15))
 (segment (start 102.148 65.15) (end 99.306 62.308) (width 0.15) (layer "F.Cu") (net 15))
 (segment (start 85.891018 49.023002) (end 85.774867 49.139156) (width 0.15) (layer "F.Cu") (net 15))
 (segment (start 85.916022 48.998007) (end 85.916016 48.998007) (width 0.15) (layer "F.Cu") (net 15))
 (segment (start 85.891022 49.023001) (end 85.891018 49.023002) (width 0.15) (layer "F.Cu") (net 15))
 (segment (start 85.685408 49.22861) (end 85.685408 49.228615) (width 0.15) (layer "F.Cu") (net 15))
 (segment (start 99.306 52.698637) (end 95.409363 48.802) (width 0.15) (layer "F.Cu") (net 15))
 (segment (start 85.916016 48.998007) (end 85.891022 49.023001) (width 0.15) (layer "F.Cu") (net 15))
 (segment (start 84.898 55.249) (end 85.674 56.025) (width 0.15) (layer "F.Cu") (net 15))
 (segment (start 85.774867 49.139156) (end 85.685408 49.22861) (width 0.15) (layer "F.Cu") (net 15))
 (segment (start 84.898 50.016025) (end 84.898 55.249) (width 0.15) (layer "F.Cu") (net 15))
 (segment (start 86.112029 48.802) (end 85.916022 48.998007) (width 0.15) (layer "F.Cu") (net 15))
 (segment (start 85.685408 49.228615) (end 84.898 50.016025) (width 0.15) (layer "F.Cu") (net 15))
 (segment (start 85.299 67.886413) (end 85.299 69.665) (width 0.15) (layer "F.Cu") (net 4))
 (segment (start 102.9 70.65) (end 98.464587 70.65) (width 0.15) (layer "F.Cu") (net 4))
 (segment (start 86.011413 67.174) (end 85.299 67.886413) (width 0.15) (layer "F.Cu") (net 4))
 (segment (start 98.464587 70.65) (end 94.988587 67.174) (width 0.15) (layer "F.Cu") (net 4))
 (segment (start 85.299 69.665) (end 85.674 70.04) (width 0.15) (layer "F.Cu") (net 4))
 (segment (start 94.988587 67.174) (end 86.011413 67.174) (width 0.15) (layer "F.Cu") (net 4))
 (segment (start 98.453751 69.15) (end 95.424751 66.121) (width 0.15) (layer "F.Cu") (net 7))
 (segment (start 84.246 67.450249) (end 84.246 77.502) (width 0.15) (layer "F.Cu") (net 7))
 (segment (start 102.9 69.15) (end 98.453751 69.15) (width 0.15) (layer "F.Cu") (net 7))
 (segment (start 85.575248 66.121) (end 84.246 67.450249) (width 0.15) (layer "F.Cu") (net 7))
 (segment (start 95.424751 66.121) (end 85.575248 66.121) (width 0.15) (layer "F.Cu") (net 7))
 (segment (start 84.246 77.502) (end 85.674 78.93) (width 0.15) (layer "F.Cu") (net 7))
 (segment (start 102.125 67.65) (end 97.551 63.076) (width 0.15) (layer "F.Cu") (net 10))
 (segment (start 97.551 63.076) (end 97.551 59.525) (width 0.15) (layer "F.Cu") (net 10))
 (segment (start 102.9 67.65) (end 102.125 67.65) (width 0.15) (layer "F.Cu") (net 10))
 (segment (start 97.551 59.525) (end 95.326 57.3) (width 0.15) (layer "F.Cu") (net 10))
 (segment (start 84.983412 48.937823) (end 84.983412 48.937829) (width 0.15) (layer "F.Cu") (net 17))
 (segment (start 85.076874 48.844361) (end 84.983416 48.937814) (width 0.15) (layer "F.Cu") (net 17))
 (segment (start 84.983408 48.937837) (end 84.196 49.725249) (width 0.15) (layer "F.Cu") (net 17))
 (segment (start 102.9 64.15) (end 102.148 64.15) (width 0.15) (layer "F.Cu") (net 17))
 (segment (start 85.625224 48.296012) (end 85.189029 48.732212) (width 0.15) (layer "F.Cu") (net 17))
 (segment (start 100.008 52.40786) (end 95.700139 48.099999) (width 0.15) (layer "F.Cu") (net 17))
 (segment (start 84.983416 48.937814) (end 84.983416 48.937819) (width 0.15) (layer "F.Cu") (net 17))
 (segment (start 85.189029 48.732212) (end 85.189023 48.732212) (width 0.15) (layer "F.Cu") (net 17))
 (segment (start 95.700139 48.099999) (end 85.821256 48.099999) (width 0.15) (layer "F.Cu") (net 17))
 (segment (start 84.983412 48.937829) (end 84.983408 48.937837) (width 0.15) (layer "F.Cu") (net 17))
 (segment (start 102.148 64.15) (end 100.008 62.01) (width 0.15) (layer "F.Cu") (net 17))
 (segment (start 85.625257 48.295997) (end 85.625233 48.296012) (width 0.15) (layer "F.Cu") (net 17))
 (segment (start 85.821256 48.099999) (end 85.625257 48.295997) (width 0.15) (layer "F.Cu") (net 17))
 (segment (start 85.625233 48.296012) (end 85.625224 48.296012) (width 0.15) (layer "F.Cu") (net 17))
 (segment (start 84.196 49.725249) (end 84.196 59.627) (width 0.15) (layer "F.Cu") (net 17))
 (segment (start 85.189023 48.732212) (end 85.076874 48.844361) (width 0.15) (layer "F.Cu") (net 17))
 (segment (start 100.008 62.01) (end 100.008 52.40786) (width 0.15) (layer "F.Cu") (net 17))
 (segment (start 84.196 59.627) (end 85.674 61.105) (width 0.15) (layer "F.Cu") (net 17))
 (segment (start 84.983416 48.937819) (end 84.983412 48.937823) (width 0.15) (layer "F.Cu") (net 17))
 (segment (start 97.2 63.3) (end 97.2 61.8) (width 0.15) (layer "F.Cu") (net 9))
 (segment (start 97.2 61.8) (end 96.51 61.11) (width 0.15) (layer "F.Cu") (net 9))
 (segment (start 102.9 68.15) (end 102.05 68.15) (width 0.15) (layer "F.Cu") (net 9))
 (segment (start 96.51 61.11) (end 95.326 61.11) (width 0.15) (layer "F.Cu") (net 9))
 (segment (start 102.05 68.15) (end 97.2 63.3) (width 0.15) (layer "F.Cu") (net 9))
 (segment (start 98.253 57.053) (end 96.4 55.2) (width 0.15) (layer "F.Cu") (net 12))
 (segment (start 95.326 52.22) (end 95.326 52.2) (width 0.15) (layer "F.Cu") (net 12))
 (segment (start 96.4 55.2) (end 96.4 52.9) (width 0.15) (layer "F.Cu") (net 12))
 (segment (start 96.4 52.9) (end 95.72 52.22) (width 0.15) (layer "F.Cu") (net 12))
 (segment (start 95.72 52.22) (end 95.326 52.22) (width 0.15) (layer "F.Cu") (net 12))
 (segment (start 98.253 62.706612) (end 98.253 57.053) (width 0.15) (layer "F.Cu") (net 12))
 (segment (start 102.196388 66.65) (end 98.253 62.706612) (width 0.15) (layer "F.Cu") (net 12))
 (segment (start 102.9 66.65) (end 102.196388 66.65) (width 0.15) (layer "F.Cu") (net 12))
 (segment (start 102.9 67.15) (end 102.2 67.15) (width 0.15) (layer "F.Cu") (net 11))
 (segment (start 97.902 58.606) (end 95.326 56.03) (width 0.15) (layer "F.Cu") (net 11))
 (segment (start 97.902 62.852) (end 97.902 58.606) (width 0.15) (layer "F.Cu") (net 11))
 (segment (start 102.2 67.15) (end 97.902 62.852) (width 0.15) (layer "F.Cu") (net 11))
 (segment (start 102.9 70.15) (end 98.460975 70.15) (width 0.15) (layer "F.Cu") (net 5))
 (segment (start 95.133975 66.823) (end 85.866025 66.823) (width 0.15) (layer "F.Cu") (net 5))
 (segment (start 98.460975 70.15) (end 95.133975 66.823) (width 0.15) (layer "F.Cu") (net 5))
 (segment (start 84.948 67.741025) (end 84.948 73.124) (width 0.15) (layer "F.Cu") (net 5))
 (segment (start 84.948 73.124) (end 85.674 73.85) (width 0.15) (layer "F.Cu") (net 5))
 (segment (start 85.866025 66.823) (end 84.948 67.741025) (width 0.15) (layer "F.Cu") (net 5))
 (segment (start 102.9 65.65) (end 102.148 65.65) (width 0.15) (layer "F.Cu") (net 14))
 (segment (start 98.955 62.457) (end 98.955 52.844026) (width 0.15) (layer "F.Cu") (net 14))
 (segment (start 102.148 65.65) (end 98.955 62.457) (width 0.15) (layer "F.Cu") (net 14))
 (segment (start 86.257419 49.153001) (end 86.061413 49.349007) (width 0.15) (layer "F.Cu") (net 14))
 (segment (start 86.061413 49.349007) (end 86.061405 49.349008) (width 0.15) (layer "F.Cu") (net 14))
 (segment (start 85.249 51.79) (end 85.674 52.215) (width 0.15) (layer "F.Cu") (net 14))
 (segment (start 86.061405 49.349008) (end 85.249 50.161413) (width 0.15) (layer "F.Cu") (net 14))
 (segment (start 98.955 52.844026) (end 95.263975 49.153001) (width 0.15) (layer "F.Cu") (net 14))
 (segment (start 95.263975 49.153001) (end 86.257419 49.153001) (width 0.15) (layer "F.Cu") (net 14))
 (segment (start 85.249 50.161413) (end 85.249 51.79) (width 0.15) (layer "F.Cu") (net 14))
 (segment (start 102.9 69.65) (end 98.457363 69.65) (width 0.15) (layer "F.Cu") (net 6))
 (segment (start 98.457363 69.65) (end 95.279363 66.472) (width 0.15) (layer "F.Cu") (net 6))
 (segment (start 85.720637 66.472) (end 84.597 67.595637) (width 0.15) (layer "F.Cu") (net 6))
 (segment (start 84.597 67.595637) (end 84.597 74.497) (width 0.15) (layer "F.Cu") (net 6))
 (segment (start 85.22 75.12) (end 85.674 75.12) (width 0.15) (layer "F.Cu") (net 6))
 (segment (start 84.597 74.497) (end 85.22 75.12) (width 0.15) (layer "F.Cu") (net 6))
 (segment (start 95.279363 66.472) (end 85.720637 66.472) (width 0.15) (layer "F.Cu") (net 6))
 (segment (start 104 63) (end 103.85 63.15) (width 0.15) (layer "F.Cu") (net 19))
 (segment (start 103.85 63.15) (end 102.9 63.15) (width 0.15) (layer "F.Cu") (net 19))
 (via (at 104 63) (size 0.6) (drill 0.3) (layers "F.Cu" "B.Cu") (free yes) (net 19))
 (segment (start 95.864587 63) (end 94.988587 63.876) (width 0.15) (layer "B.Cu") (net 19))
 (segment (start 104 63) (end 95.864587 63) (width 0.15) (layer "B.Cu") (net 19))
 (segment (start 94.988587 63.876) (end 75.362 63.876) (width 0.15) (layer "B.Cu") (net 19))
 (segment (start 75.362 63.876) (end 71.326 59.84) (width 0.15) (layer "B.Cu") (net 19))
 (segment (start 102.9 59.65) (end 103.85 59.65) (width 0.15) (layer "F.Cu") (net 23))
 (segment (start 107.8 80.1) (end 108.5 80.1) (width 0.6) (layers "F.Cu" "F.Mask") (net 23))
 (segment (start 103.85 59.65) (end 104 59.5) (width 0.15) (layer "F.Cu") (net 23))
 (via (at 107.8 80.1) (size 0.6) (drill 0.3) (layers "F.Cu" "B.Cu") (free yes) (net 23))
 (via (at 104 59.5) (size 0.6) (drill 0.3) (layers "F.Cu" "B.Cu") (free yes) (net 23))
 (segment (start 107.8 80.1) (end 108.8 79.1) (width 0.15) (layer "B.Cu") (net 23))
 (segment (start 108.8 79.1) (end 108.8 76.6) (width 0.15) (layer "B.Cu") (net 23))
 (segment (start 107.4 75.2) (end 107.4 62.885412) (width 0.15) (layer "B.Cu") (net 23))
 (segment (start 104.014588 59.5) (end 104 59.5) (width 0.15) (layer "B.Cu") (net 23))
 (segment (start 107.4 62.885412) (end 104.014588 59.5) (width 0.15) (layer "B.Cu") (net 23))
 (segment (start 108.8 76.6) (end 107.4 75.2) (width 0.15) (layer "B.Cu") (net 23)))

